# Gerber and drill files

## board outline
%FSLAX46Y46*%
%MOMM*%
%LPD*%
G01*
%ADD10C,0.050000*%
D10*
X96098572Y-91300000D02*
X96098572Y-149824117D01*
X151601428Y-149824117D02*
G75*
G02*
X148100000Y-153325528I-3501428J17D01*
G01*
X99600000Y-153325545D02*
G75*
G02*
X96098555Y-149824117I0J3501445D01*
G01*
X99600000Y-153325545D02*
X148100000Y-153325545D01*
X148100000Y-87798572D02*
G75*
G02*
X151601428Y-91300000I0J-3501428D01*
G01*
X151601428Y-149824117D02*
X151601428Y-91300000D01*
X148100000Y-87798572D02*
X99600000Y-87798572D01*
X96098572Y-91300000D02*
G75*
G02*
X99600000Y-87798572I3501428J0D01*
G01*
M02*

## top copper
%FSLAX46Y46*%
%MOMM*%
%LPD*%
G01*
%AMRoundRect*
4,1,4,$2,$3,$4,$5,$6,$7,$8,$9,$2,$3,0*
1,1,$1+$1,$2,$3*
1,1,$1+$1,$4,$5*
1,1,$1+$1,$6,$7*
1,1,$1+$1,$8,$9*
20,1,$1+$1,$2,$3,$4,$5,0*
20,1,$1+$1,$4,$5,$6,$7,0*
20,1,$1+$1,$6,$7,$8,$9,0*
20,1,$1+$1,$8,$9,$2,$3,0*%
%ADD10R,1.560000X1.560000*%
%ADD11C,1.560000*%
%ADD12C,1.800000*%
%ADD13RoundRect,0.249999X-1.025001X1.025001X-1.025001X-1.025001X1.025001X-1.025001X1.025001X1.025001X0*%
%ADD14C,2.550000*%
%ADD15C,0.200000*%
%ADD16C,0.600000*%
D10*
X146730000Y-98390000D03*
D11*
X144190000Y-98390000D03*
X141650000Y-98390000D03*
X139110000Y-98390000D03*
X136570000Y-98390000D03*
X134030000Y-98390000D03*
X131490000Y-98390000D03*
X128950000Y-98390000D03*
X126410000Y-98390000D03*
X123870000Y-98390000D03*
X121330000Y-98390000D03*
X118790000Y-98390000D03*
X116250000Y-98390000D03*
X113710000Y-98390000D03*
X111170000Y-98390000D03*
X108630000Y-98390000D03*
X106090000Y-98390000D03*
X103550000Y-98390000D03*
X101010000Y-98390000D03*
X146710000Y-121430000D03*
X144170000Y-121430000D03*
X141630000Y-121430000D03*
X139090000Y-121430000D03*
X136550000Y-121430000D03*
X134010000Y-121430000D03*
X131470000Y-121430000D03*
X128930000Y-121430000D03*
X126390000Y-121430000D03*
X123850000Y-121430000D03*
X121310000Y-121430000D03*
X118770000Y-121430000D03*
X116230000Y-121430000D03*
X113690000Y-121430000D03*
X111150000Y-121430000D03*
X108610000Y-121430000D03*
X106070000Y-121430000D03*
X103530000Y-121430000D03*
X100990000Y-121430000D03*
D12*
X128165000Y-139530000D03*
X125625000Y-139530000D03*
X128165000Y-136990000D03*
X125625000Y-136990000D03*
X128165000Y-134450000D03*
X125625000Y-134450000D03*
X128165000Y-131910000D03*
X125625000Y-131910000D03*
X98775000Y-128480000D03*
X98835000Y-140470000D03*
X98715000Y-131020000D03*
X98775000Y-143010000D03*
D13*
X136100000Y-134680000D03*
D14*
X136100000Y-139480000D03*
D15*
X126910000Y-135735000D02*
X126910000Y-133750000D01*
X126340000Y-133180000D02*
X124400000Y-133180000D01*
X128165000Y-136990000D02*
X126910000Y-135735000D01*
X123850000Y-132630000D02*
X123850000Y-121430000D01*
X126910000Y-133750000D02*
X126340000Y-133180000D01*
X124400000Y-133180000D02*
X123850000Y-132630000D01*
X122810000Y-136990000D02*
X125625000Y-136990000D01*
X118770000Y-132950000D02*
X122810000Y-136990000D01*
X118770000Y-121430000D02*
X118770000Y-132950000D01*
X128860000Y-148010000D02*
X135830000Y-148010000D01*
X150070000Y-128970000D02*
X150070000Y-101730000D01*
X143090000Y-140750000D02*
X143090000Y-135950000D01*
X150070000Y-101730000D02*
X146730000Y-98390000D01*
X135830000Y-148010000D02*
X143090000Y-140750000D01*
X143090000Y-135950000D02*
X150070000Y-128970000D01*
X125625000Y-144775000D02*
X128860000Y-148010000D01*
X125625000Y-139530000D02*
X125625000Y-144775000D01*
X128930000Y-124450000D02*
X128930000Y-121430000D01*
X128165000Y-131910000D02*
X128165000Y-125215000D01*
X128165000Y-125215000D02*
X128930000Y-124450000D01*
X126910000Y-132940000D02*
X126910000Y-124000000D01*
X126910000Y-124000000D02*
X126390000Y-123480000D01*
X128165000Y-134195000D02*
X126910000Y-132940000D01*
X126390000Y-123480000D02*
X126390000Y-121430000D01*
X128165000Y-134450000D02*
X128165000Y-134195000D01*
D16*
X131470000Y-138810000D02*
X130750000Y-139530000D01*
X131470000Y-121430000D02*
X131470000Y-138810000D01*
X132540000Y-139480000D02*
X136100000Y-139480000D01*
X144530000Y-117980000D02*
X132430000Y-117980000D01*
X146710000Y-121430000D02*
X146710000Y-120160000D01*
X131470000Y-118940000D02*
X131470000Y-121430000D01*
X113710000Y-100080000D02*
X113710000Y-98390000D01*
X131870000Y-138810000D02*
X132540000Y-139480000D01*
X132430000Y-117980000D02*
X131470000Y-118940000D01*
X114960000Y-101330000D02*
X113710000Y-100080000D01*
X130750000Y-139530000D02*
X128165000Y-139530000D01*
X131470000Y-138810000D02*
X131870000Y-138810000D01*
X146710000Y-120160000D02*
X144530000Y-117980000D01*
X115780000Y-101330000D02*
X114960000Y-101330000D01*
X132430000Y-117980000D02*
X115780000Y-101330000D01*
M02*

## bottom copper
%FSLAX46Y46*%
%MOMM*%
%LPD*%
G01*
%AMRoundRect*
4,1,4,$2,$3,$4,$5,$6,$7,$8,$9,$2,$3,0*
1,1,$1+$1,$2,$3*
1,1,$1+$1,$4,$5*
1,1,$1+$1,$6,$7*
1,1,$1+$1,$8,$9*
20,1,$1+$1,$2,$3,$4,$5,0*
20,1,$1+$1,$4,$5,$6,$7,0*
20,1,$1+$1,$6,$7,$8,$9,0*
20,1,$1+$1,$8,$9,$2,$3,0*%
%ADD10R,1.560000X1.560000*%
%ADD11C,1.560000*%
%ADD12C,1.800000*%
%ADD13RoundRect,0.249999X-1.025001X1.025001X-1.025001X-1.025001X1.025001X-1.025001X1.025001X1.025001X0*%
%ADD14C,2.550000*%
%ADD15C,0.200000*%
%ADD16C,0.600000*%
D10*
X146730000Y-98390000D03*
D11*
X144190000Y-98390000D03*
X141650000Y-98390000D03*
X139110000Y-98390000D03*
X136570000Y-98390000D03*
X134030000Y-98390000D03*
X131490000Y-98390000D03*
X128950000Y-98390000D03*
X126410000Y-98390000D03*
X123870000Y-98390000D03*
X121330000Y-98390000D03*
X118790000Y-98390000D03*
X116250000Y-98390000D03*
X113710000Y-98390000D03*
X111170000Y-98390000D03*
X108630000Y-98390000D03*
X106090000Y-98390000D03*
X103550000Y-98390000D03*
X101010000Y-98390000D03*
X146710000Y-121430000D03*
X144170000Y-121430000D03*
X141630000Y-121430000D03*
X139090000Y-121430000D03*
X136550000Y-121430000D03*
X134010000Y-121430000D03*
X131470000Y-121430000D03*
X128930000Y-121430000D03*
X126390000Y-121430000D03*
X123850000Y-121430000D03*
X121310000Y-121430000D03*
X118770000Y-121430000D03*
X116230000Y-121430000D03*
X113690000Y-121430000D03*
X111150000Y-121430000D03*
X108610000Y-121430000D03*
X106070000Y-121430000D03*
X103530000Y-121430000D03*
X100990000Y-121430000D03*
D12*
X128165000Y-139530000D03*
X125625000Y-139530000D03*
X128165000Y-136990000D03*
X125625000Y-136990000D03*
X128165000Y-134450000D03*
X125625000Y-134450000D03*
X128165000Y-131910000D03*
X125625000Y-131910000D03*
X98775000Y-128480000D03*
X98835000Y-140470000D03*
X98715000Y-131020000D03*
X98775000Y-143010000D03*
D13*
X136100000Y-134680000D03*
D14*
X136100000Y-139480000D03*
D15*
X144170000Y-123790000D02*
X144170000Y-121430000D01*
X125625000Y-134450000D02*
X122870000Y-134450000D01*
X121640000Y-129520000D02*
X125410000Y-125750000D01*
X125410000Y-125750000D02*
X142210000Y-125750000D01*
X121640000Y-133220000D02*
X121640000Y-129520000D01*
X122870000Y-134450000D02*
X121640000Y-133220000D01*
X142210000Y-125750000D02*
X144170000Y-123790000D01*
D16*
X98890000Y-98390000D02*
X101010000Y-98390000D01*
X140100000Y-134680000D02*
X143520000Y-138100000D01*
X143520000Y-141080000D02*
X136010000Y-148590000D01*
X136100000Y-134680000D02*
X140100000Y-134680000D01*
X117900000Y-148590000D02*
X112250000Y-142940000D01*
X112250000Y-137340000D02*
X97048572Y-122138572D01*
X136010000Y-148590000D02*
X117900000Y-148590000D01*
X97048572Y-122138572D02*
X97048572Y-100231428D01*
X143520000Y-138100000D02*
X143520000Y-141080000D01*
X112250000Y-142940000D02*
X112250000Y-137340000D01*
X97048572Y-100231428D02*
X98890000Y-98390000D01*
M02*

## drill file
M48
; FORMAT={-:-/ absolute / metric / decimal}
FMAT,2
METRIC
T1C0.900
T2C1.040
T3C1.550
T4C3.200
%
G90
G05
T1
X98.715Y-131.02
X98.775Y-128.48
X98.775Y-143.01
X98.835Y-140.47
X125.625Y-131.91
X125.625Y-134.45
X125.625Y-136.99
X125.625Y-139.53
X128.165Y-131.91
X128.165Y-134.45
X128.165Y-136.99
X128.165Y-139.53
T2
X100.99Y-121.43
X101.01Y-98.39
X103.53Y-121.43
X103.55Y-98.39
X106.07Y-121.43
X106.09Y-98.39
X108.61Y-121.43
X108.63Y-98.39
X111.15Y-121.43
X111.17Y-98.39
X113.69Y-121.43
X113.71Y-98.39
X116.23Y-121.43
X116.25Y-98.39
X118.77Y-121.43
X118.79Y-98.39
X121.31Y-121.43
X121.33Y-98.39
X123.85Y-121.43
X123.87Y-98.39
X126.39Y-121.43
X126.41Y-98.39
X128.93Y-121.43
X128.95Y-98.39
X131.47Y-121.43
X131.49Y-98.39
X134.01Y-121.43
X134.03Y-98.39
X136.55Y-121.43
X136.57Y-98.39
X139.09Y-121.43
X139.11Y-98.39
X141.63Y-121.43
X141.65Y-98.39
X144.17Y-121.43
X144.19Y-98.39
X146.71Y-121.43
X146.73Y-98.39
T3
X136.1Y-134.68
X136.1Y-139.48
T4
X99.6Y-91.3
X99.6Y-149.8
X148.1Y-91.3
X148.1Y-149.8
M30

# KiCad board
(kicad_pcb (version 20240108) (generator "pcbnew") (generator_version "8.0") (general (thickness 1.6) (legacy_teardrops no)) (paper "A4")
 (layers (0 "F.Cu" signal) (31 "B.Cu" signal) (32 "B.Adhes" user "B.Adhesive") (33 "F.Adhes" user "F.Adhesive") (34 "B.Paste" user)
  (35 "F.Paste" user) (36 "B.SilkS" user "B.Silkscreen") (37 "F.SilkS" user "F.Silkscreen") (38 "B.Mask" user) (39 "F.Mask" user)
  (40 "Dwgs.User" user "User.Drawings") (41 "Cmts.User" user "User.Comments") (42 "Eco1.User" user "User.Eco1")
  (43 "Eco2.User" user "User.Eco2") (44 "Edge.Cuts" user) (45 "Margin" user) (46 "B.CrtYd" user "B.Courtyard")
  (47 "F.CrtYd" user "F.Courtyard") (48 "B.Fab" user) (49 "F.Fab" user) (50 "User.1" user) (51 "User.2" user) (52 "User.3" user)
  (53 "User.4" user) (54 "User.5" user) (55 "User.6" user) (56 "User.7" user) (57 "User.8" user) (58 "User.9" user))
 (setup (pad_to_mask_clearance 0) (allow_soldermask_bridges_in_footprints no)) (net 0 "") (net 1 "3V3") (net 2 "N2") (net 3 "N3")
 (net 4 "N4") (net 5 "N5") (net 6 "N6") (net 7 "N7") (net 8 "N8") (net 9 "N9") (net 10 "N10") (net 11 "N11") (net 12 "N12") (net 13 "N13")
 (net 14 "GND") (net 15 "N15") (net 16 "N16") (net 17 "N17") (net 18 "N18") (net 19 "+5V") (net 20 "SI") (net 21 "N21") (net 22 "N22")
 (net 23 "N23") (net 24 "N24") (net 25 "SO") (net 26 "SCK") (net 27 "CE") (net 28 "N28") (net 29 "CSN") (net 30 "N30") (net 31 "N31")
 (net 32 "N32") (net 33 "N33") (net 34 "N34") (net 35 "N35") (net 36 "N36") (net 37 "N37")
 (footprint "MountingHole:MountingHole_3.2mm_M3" (layer "F.Cu") (at 148.1 91.3 180)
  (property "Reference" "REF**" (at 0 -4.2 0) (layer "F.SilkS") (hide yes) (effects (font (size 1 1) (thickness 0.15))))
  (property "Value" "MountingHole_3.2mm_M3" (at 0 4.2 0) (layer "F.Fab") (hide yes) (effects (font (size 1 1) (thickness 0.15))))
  (pad "" np_thru_hole circle (at 0 0 180) (size 3.2 3.2) (drill 3.2) (layers "*.Cu" "*.Mask")))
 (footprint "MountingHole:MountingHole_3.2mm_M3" (layer "F.Cu") (at 99.6 91.3 180)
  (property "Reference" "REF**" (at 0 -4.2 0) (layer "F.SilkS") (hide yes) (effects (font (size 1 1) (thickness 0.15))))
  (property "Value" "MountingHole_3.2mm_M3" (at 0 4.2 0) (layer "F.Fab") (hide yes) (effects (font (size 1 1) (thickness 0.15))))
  (pad "" np_thru_hole circle (at 0 0 180) (size 3.2 3.2) (drill 3.2) (layers "*.Cu" "*.Mask")))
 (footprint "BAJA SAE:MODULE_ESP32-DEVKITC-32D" (layer "F.Cu") (at 127.8 110.15 -90)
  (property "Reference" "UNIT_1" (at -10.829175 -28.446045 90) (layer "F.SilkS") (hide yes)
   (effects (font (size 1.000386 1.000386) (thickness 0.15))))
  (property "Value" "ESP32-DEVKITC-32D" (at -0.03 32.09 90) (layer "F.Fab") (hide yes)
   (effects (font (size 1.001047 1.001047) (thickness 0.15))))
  (pad "J2-1" thru_hole rect (at -11.76 -18.93 270) (size 1.56 1.56) (drill 1.04) (layers "*.Cu" "*.Mask") (remove_unused_layers no)
   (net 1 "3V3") (solder_mask_margin 0.102))
  (pad "J2-2" thru_hole circle (at -11.76 -16.39 270) (size 1.56 1.56) (drill 1.04) (layers "*.Cu" "*.Mask") (remove_unused_layers no)
   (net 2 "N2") (solder_mask_margin 0.102))
  (pad "J2-3" thru_hole circle (at -11.76 -13.85 270) (size 1.56 1.56) (drill 1.04) (layers "*.Cu" "*.Mask") (remove_unused_layers no)
   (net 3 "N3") (solder_mask_margin 0.102))
  (pad "J2-4" thru_hole circle (at -11.76 -11.31 270) (size 1.56 1.56) (drill 1.04) (layers "*.Cu" "*.Mask") (remove_unused_layers no)
   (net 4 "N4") (solder_mask_margin 0.102))
  (pad "J2-5" thru_hole circle (at -11.76 -8.77 270) (size 1.56 1.56) (drill 1.04) (layers "*.Cu" "*.Mask") (remove_unused_layers no)
   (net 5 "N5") (solder_mask_margin 0.102))
  (pad "J2-6" thru_hole circle (at -11.76 -6.23 270) (size 1.56 1.56) (drill 1.04) (layers "*.Cu" "*.Mask") (remove_unused_layers no)
   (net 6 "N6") (solder_mask_margin 0.102))
  (pad "J2-7" thru_hole circle (at -11.76 -3.69 270) (size 1.56 1.56) (drill 1.04) (layers "*.Cu" "*.Mask") (remove_unused_layers no)
   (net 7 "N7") (solder_mask_margin 0.102))
  (pad "J2-8" thru_hole circle (at -11.76 -1.15 270) (size 1.56 1.56) (drill 1.04) (layers "*.Cu" "*.Mask") (remove_unused_layers no)
   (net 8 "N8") (solder_mask_margin 0.102))
  (pad "J2-9" thru_hole circle (at -11.76 1.39 270) (size 1.56 1.56) (drill 1.04) (layers "*.Cu" "*.Mask") (remove_unused_layers no)
   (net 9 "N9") (solder_mask_margin 0.102))
  (pad "J2-10" thru_hole circle (at -11.76 3.93 270) (size 1.56 1.56) (drill 1.04) (layers "*.Cu" "*.Mask") (remove_unused_layers no)
   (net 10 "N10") (solder_mask_margin 0.102))
  (pad "J2-11" thru_hole circle (at -11.76 6.47 270) (size 1.56 1.56) (drill 1.04) (layers "*.Cu" "*.Mask") (remove_unused_layers no)
   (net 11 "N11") (solder_mask_margin 0.102))
  (pad "J2-12" thru_hole circle (at -11.76 9.01 270) (size 1.56 1.56) (drill 1.04) (layers "*.Cu" "*.Mask") (remove_unused_layers no)
   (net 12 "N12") (solder_mask_margin 0.102))
  (pad "J2-13" thru_hole circle (at -11.76 11.55 270) (size 1.56 1.56) (drill 1.04) (layers "*.Cu" "*.Mask") (remove_unused_layers no)
   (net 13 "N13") (solder_mask_margin 0.102))
  (pad "J2-14" thru_hole circle (at -11.76 14.09 270) (size 1.56 1.56) (drill 1.04) (layers "*.Cu" "*.Mask") (remove_unused_layers no)
   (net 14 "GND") (solder_mask_margin 0.102))
  (pad "J2-15" thru_hole circle (at -11.76 16.63 270) (size 1.56 1.56) (drill 1.04) (layers "*.Cu" "*.Mask") (remove_unused_layers no)
   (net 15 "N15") (solder_mask_margin 0.102))
  (pad "J2-16" thru_hole circle (at -11.76 19.17 270) (size 1.56 1.56) (drill 1.04) (layers "*.Cu" "*.Mask") (remove_unused_layers no)
   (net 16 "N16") (solder_mask_margin 0.102))
  (pad "J2-17" thru_hole circle (at -11.76 21.71 270) (size 1.56 1.56) (drill 1.04) (layers "*.Cu" "*.Mask") (remove_unused_layers no)
   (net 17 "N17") (solder_mask_margin 0.102))
  (pad "J2-18" thru_hole circle (at -11.76 24.25 270) (size 1.56 1.56) (drill 1.04) (layers "*.Cu" "*.Mask") (remove_unused_layers no)
   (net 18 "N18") (solder_mask_margin 0.102))
  (pad "J2-19" thru_hole circle (at -11.76 26.79 270) (size 1.56 1.56) (drill 1.04) (layers "*.Cu" "*.Mask") (remove_unused_layers no)
   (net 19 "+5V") (solder_mask_margin 0.102))
  (pad "J3-1" thru_hole circle (at 11.28 -18.91 270) (size 1.56 1.56) (drill 1.04) (layers "*.Cu" "*.Mask") (remove_unused_layers no)
   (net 14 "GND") (solder_mask_margin 0.102))
  (pad "J3-2" thru_hole circle (at 11.28 -16.37 270) (size 1.56 1.56) (drill 1.04) (layers "*.Cu" "*.Mask") (remove_unused_layers no)
   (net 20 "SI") (solder_mask_margin 0.102))
  (pad "J3-3" thru_hole circle (at 11.28 -13.83 270) (size 1.56 1.56) (drill 1.04) (layers "*.Cu" "*.Mask") (remove_unused_layers no)
   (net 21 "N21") (solder_mask_margin 0.102))
  (pad "J3-4" thru_hole circle (at 11.28 -11.29 270) (size 1.56 1.56) (drill 1.04) (layers "*.Cu" "*.Mask") (remove_unused_layers no)
   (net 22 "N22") (solder_mask_margin 0.102))
  (pad "J3-5" thru_hole circle (at 11.28 -8.75 270) (size 1.56 1.56) (drill 1.04) (layers "*.Cu" "*.Mask") (remove_unused_layers no)
   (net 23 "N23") (solder_mask_margin 0.102))
  (pad "J3-6" thru_hole circle (at 11.28 -6.21 270) (size 1.56 1.56) (drill 1.04) (layers "*.Cu" "*.Mask") (remove_unused_layers no)
   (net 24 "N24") (solder_mask_margin 0.102))
  (pad "J3-7" thru_hole circle (at 11.28 -3.67 270) (size 1.56 1.56) (drill 1.04) (layers "*.Cu" "*.Mask") (remove_unused_layers no)
   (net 14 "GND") (solder_mask_margin 0.102))
  (pad "J3-8" thru_hole circle (at 11.28 -1.13 270) (size 1.56 1.56) (drill 1.04) (layers "*.Cu" "*.Mask") (remove_unused_layers no)
   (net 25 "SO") (solder_mask_margin 0.102))
  (pad "J3-9" thru_hole circle (at 11.28 1.41 270) (size 1.56 1.56) (drill 1.04) (layers "*.Cu" "*.Mask") (remove_unused_layers no)
   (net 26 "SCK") (solder_mask_margin 0.102))
  (pad "J3-10" thru_hole circle (at 11.28 3.95 270) (size 1.56 1.56) (drill 1.04) (layers "*.Cu" "*.Mask") (remove_unused_layers no)
   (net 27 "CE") (solder_mask_margin 0.102))
  (pad "J3-11" thru_hole circle (at 11.28 6.49 270) (size 1.56 1.56) (drill 1.04) (layers "*.Cu" "*.Mask") (remove_unused_layers no)
   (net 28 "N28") (solder_mask_margin 0.102))
  (pad "J3-12" thru_hole circle (at 11.28 9.03 270) (size 1.56 1.56) (drill 1.04) (layers "*.Cu" "*.Mask") (remove_unused_layers no)
   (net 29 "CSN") (solder_mask_margin 0.102))
  (pad "J3-13" thru_hole circle (at 11.28 11.57 270) (size 1.56 1.56) (drill 1.04) (layers "*.Cu" "*.Mask") (remove_unused_layers no)
   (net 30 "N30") (solder_mask_margin 0.102))
  (pad "J3-14" thru_hole circle (at 11.28 14.11 270) (size 1.56 1.56) (drill 1.04) (layers "*.Cu" "*.Mask") (remove_unused_layers no)
   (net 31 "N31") (solder_mask_margin 0.102))
  (pad "J3-15" thru_hole circle (at 11.28 16.65 270) (size 1.56 1.56) (drill 1.04) (layers "*.Cu" "*.Mask") (remove_unused_layers no)
   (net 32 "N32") (solder_mask_margin 0.102))
  (pad "J3-16" thru_hole circle (at 11.28 19.19 270) (size 1.56 1.56) (drill 1.04) (layers "*.Cu" "*.Mask") (remove_unused_layers no)
   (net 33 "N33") (solder_mask_margin 0.102))
  (pad "J3-17" thru_hole circle (at 11.28 21.73 270) (size 1.56 1.56) (drill 1.04) (layers "*.Cu" "*.Mask") (remove_unused_layers no)
   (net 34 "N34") (solder_mask_margin 0.102))
  (pad "J3-18" thru_hole circle (at 11.28 24.27 270) (size 1.56 1.56) (drill 1.04) (layers "*.Cu" "*.Mask") (remove_unused_layers no)
   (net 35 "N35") (solder_mask_margin 0.102))
  (pad "J3-19" thru_hole circle (at 11.28 26.81 270) (size 1.56 1.56) (drill 1.04) (layers "*.Cu" "*.Mask") (remove_unused_layers no)
   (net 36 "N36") (solder_mask_margin 0.102)))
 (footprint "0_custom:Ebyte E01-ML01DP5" (layer "F.Cu") (at 132.985 135.7 -90)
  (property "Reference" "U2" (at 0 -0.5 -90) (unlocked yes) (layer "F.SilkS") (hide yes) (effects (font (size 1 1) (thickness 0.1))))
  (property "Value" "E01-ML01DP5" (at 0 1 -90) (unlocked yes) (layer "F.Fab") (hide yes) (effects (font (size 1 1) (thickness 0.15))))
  (pad "1" thru_hole circle (at 3.83 4.82 90) (size 1.8 1.8) (drill 0.9) (layers "*.Cu" "*.Mask") (remove_unused_layers no) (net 14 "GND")
   (solder_mask_margin 0.102))
  (pad "2" thru_hole circle (at 3.83 7.36 90) (size 1.8 1.8) (drill 0.9) (layers "*.Cu" "*.Mask") (remove_unused_layers no) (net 1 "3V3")
   (solder_mask_margin 0.102))
  (pad "3" thru_hole circle (at 1.29 4.82 90) (size 1.8 1.8) (drill 0.9) (layers "*.Cu" "*.Mask") (remove_unused_layers no) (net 27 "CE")
   (solder_mask_margin 0.102))
  (pad "4" thru_hole circle (at 1.29 7.36 90) (size 1.8 1.8) (drill 0.9) (layers "*.Cu" "*.Mask") (remove_unused_layers no) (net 29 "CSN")
   (solder_mask_margin 0.102))
  (pad "5" thru_hole circle (at -1.25 4.82 90) (size 1.8 1.8) (drill 0.9) (layers "*.Cu" "*.Mask") (remove_unused_layers no) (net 26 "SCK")
   (solder_mask_margin 0.102))
  (pad "6" thru_hole circle (at -1.25 7.36 90) (size 1.8 1.8) (drill 0.9) (layers "*.Cu" "*.Mask") (remove_unused_layers no) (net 20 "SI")
   (solder_mask_margin 0.102))
  (pad "7" thru_hole circle (at -3.79 4.82) (size 1.8 1.8) (drill 0.9) (layers "*.Cu" "*.Mask") (remove_unused_layers no) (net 25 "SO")
   (solder_mask_margin 0.102))
  (pad "8" thru_hole circle (at -3.79 7.36) (size 1.8 1.8) (drill 0.9) (layers "*.Cu" "*.Mask") (remove_unused_layers no) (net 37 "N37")
   (solder_mask_margin 0.102))
  (pad "9" thru_hole circle (at -7.22 34.21 180) (size 1.8 1.8) (drill 0.9) (layers "*.Cu" "*.Mask") (remove_unused_layers no)
   (solder_mask_margin 0.102))
  (pad "9" thru_hole circle (at 4.77 34.15 180) (size 1.8 1.8) (drill 0.9) (layers "*.Cu" "*.Mask") (remove_unused_layers no)
   (solder_mask_margin 0.102))
  (pad "10" thru_hole circle (at -4.68 34.27 180) (size 1.8 1.8) (drill 0.9) (layers "*.Cu" "*.Mask") (remove_unused_layers no)
   (solder_mask_margin 0.102))
  (pad "10" thru_hole circle (at 7.31 34.21 180) (size 1.8 1.8) (drill 0.9) (layers "*.Cu" "*.Mask") (remove_unused_layers no)
   (solder_mask_margin 0.102)))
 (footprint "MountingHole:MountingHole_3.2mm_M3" (layer "F.Cu") (at 99.6 149.8)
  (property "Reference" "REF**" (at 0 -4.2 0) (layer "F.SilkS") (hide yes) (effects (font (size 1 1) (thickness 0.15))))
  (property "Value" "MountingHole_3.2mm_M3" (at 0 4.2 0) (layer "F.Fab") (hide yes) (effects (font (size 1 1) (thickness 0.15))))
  (pad "" np_thru_hole circle (at 0 0) (size 3.2 3.2) (drill 3.2) (layers "*.Cu" "*.Mask")))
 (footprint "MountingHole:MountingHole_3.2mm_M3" (layer "F.Cu") (at 148.1 149.8)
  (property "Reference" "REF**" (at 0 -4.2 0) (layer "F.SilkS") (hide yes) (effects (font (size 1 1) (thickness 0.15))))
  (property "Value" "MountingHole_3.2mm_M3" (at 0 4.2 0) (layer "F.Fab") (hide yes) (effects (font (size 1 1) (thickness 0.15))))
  (pad "" np_thru_hole circle (at 0 0) (size 3.2 3.2) (drill 3.2) (layers "*.Cu" "*.Mask")))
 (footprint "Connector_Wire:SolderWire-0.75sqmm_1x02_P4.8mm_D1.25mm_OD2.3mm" (layer "F.Cu") (at 136.1 134.68 -90)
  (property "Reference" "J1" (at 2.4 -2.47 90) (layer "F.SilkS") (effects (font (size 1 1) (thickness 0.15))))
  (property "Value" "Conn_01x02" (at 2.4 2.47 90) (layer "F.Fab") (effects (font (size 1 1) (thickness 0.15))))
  (pad "1" thru_hole roundrect (at 0 0 270) (size 2.55 2.55) (drill 1.55) (layers "*.Cu" "*.Mask") (remove_unused_layers no)
   (roundrect_rratio 0.098039) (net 19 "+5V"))
  (pad "2" thru_hole circle (at 4.8 0 270) (size 2.55 2.55) (drill 1.55) (layers "*.Cu" "*.Mask") (remove_unused_layers no) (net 14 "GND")))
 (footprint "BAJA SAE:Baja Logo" (layer "B.Cu") (at 124.22 104.45 180)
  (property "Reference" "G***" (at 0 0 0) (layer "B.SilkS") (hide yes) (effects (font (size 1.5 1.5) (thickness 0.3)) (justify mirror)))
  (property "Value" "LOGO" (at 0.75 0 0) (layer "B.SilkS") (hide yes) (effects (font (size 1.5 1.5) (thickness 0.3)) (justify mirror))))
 (gr_line (start 96.098572 91.3) (end 96.098572 149.824117) (stroke (width 0.05) (type default)) (layer "Edge.Cuts"))
 (gr_arc (start 151.601428 149.824117) (mid 150.575883 152.3) (end 148.1 153.325545) (locked yes) (stroke (width 0.05) (type default))
  (layer "Edge.Cuts"))
 (gr_arc (start 99.6 153.325545) (mid 97.124117 152.3) (end 96.098572 149.824117) (stroke (width 0.05) (type default)) (layer "Edge.Cuts"))
 (gr_line (start 99.6 153.325545) (end 148.1 153.325545) (stroke (width 0.05) (type default)) (layer "Edge.Cuts"))
 (gr_arc (start 148.1 87.798572) (mid 150.575883 88.824117) (end 151.601428 91.3) (locked yes) (stroke (width 0.05) (type default))
  (layer "Edge.Cuts"))
 (gr_line (start 151.601428 149.824117) (end 151.601428 91.3) (stroke (width 0.05) (type default)) (layer "Edge.Cuts"))
 (gr_line (start 148.1 87.798572) (end 99.6 87.798572) (stroke (width 0.05) (type default)) (layer "Edge.Cuts"))
 (gr_arc (start 96.098572 91.3) (mid 97.124117 88.824117) (end 99.6 87.798572) (locked yes) (stroke (width 0.05) (type default))
  (layer "Edge.Cuts"))
 (segment (start 126.91 135.735) (end 126.91 133.75) (width 0.2) (layer "F.Cu") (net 27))
 (segment (start 126.34 133.18) (end 124.4 133.18) (width 0.2) (layer "F.Cu") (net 27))
 (segment (start 128.165 136.99) (end 126.91 135.735) (width 0.2) (layer "F.Cu") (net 27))
 (segment (start 123.85 132.63) (end 123.85 121.43) (width 0.2) (layer "F.Cu") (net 27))
 (segment (start 126.91 133.75) (end 126.34 133.18) (width 0.2) (layer "F.Cu") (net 27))
 (segment (start 124.4 133.18) (end 123.85 132.63) (width 0.2) (layer "F.Cu") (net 27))
 (segment (start 122.81 136.99) (end 125.625 136.99) (width 0.2) (layer "F.Cu") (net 29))
 (segment (start 118.77 132.95) (end 122.81 136.99) (width 0.2) (layer "F.Cu") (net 29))
 (segment (start 118.77 121.43) (end 118.77 132.95) (width 0.2) (layer "F.Cu") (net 29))
 (segment (start 128.86 148.01) (end 135.83 148.01) (width 0.2) (layer "F.Cu") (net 1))
 (segment (start 150.07 128.97) (end 150.07 101.73) (width 0.2) (layer "F.Cu") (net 1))
 (segment (start 143.09 140.75) (end 143.09 135.95) (width 0.2) (layer "F.Cu") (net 1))
 (segment (start 150.07 101.73) (end 146.73 98.39) (width 0.2) (layer "F.Cu") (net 1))
 (segment (start 135.83 148.01) (end 143.09 140.75) (width 0.2) (layer "F.Cu") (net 1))
 (segment (start 143.09 135.95) (end 150.07 128.97) (width 0.2) (layer "F.Cu") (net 1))
 (segment (start 125.625 144.775) (end 128.86 148.01) (width 0.2) (layer "F.Cu") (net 1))
 (segment (start 125.625 139.53) (end 125.625 144.775) (width 0.2) (layer "F.Cu") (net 1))
 (segment (start 128.93 124.45) (end 128.93 121.43) (width 0.2) (layer "F.Cu") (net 25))
 (segment (start 128.165 131.91) (end 128.165 125.215) (width 0.2) (layer "F.Cu") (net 25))
 (segment (start 128.165 125.215) (end 128.93 124.45) (width 0.2) (layer "F.Cu") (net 25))
 (segment (start 126.91 132.94) (end 126.91 124) (width 0.2) (layer "F.Cu") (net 26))
 (segment (start 126.91 124) (end 126.39 123.48) (width 0.2) (layer "F.Cu") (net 26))
 (segment (start 128.165 134.195) (end 126.91 132.94) (width 0.2) (layer "F.Cu") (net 26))
 (segment (start 126.39 123.48) (end 126.39 121.43) (width 0.2) (layer "F.Cu") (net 26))
 (segment (start 128.165 134.45) (end 128.165 134.195) (width 0.2) (layer "F.Cu") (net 26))
 (segment (start 144.17 123.79) (end 144.17 121.43) (width 0.2) (layer "B.Cu") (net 20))
 (segment (start 125.625 134.45) (end 122.87 134.45) (width 0.2) (layer "B.Cu") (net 20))
 (segment (start 121.64 129.52) (end 125.41 125.75) (width 0.2) (layer "B.Cu") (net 20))
 (segment (start 125.41 125.75) (end 142.21 125.75) (width 0.2) (layer "B.Cu") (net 20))
 (segment (start 121.64 133.22) (end 121.64 129.52) (width 0.2) (layer "B.Cu") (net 20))
 (segment (start 122.87 134.45) (end 121.64 133.22) (width 0.2) (layer "B.Cu") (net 20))
 (segment (start 142.21 125.75) (end 144.17 123.79) (width 0.2) (layer "B.Cu") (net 20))
 (segment (start 131.47 138.81) (end 130.75 139.53) (width 0.6) (layer "F.Cu") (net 14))
 (segment (start 131.47 121.43) (end 131.47 138.81) (width 0.6) (layer "F.Cu") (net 14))
 (segment (start 132.54 139.48) (end 136.1 139.48) (width 0.6) (layer "F.Cu") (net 14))
 (segment (start 144.53 117.98) (end 132.43 117.98) (width 0.6) (layer "F.Cu") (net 14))
 (segment (start 146.71 121.43) (end 146.71 120.16) (width 0.6) (layer "F.Cu") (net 14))
 (segment (start 131.47 118.94) (end 131.47 121.43) (width 0.6) (layer "F.Cu") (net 14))
 (segment (start 113.71 100.08) (end 113.71 98.39) (width 0.6) (layer "F.Cu") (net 14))
 (segment (start 131.87 138.81) (end 132.54 139.48) (width 0.6) (layer "F.Cu") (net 14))
 (segment (start 132.43 117.98) (end 131.47 118.94) (width 0.6) (layer "F.Cu") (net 14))
 (segment (start 114.96 101.33) (end 113.71 100.08) (width 0.6) (layer "F.Cu") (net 14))
 (segment (start 130.75 139.53) (end 128.165 139.53) (width 0.6) (layer "F.Cu") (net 14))
 (segment (start 131.47 138.81) (end 131.87 138.81) (width 0.6) (layer "F.Cu") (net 14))
 (segment (start 146.71 120.16) (end 144.53 117.98) (width 0.6) (layer "F.Cu") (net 14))
 (segment (start 115.78 101.33) (end 114.96 101.33) (width 0.6) (layer "F.Cu") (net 14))
 (segment (start 132.43 117.98) (end 115.78 101.33) (width 0.6) (layer "F.Cu") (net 14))
 (segment (start 98.89 98.39) (end 101.01 98.39) (width 0.6) (layer "B.Cu") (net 19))
 (segment (start 140.1 134.68) (end 143.52 138.1) (width 0.6) (layer "B.Cu") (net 19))
 (segment (start 143.52 141.08) (end 136.01 148.59) (width 0.6) (layer "B.Cu") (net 19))
 (segment (start 136.1 134.68) (end 140.1 134.68) (width 0.6) (layer "B.Cu") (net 19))
 (segment (start 117.9 148.59) (end 112.25 142.94) (width 0.6) (layer "B.Cu") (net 19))
 (segment (start 112.25 137.34) (end 97.048572 122.138572) (width 0.6) (layer "B.Cu") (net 19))
 (segment (start 136.01 148.59) (end 117.9 148.59) (width 0.6) (layer "B.Cu") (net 19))
 (segment (start 97.048572 122.138572) (end 97.048572 100.231428) (width 0.6) (layer "B.Cu") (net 19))
 (segment (start 143.52 138.1) (end 143.52 141.08) (width 0.6) (layer "B.Cu") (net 19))
 (segment (start 112.25 142.94) (end 112.25 137.34) (width 0.6) (layer "B.Cu") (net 19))
 (segment (start 97.048572 100.231428) (end 98.89 98.39) (width 0.6) (layer "B.Cu") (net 19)))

